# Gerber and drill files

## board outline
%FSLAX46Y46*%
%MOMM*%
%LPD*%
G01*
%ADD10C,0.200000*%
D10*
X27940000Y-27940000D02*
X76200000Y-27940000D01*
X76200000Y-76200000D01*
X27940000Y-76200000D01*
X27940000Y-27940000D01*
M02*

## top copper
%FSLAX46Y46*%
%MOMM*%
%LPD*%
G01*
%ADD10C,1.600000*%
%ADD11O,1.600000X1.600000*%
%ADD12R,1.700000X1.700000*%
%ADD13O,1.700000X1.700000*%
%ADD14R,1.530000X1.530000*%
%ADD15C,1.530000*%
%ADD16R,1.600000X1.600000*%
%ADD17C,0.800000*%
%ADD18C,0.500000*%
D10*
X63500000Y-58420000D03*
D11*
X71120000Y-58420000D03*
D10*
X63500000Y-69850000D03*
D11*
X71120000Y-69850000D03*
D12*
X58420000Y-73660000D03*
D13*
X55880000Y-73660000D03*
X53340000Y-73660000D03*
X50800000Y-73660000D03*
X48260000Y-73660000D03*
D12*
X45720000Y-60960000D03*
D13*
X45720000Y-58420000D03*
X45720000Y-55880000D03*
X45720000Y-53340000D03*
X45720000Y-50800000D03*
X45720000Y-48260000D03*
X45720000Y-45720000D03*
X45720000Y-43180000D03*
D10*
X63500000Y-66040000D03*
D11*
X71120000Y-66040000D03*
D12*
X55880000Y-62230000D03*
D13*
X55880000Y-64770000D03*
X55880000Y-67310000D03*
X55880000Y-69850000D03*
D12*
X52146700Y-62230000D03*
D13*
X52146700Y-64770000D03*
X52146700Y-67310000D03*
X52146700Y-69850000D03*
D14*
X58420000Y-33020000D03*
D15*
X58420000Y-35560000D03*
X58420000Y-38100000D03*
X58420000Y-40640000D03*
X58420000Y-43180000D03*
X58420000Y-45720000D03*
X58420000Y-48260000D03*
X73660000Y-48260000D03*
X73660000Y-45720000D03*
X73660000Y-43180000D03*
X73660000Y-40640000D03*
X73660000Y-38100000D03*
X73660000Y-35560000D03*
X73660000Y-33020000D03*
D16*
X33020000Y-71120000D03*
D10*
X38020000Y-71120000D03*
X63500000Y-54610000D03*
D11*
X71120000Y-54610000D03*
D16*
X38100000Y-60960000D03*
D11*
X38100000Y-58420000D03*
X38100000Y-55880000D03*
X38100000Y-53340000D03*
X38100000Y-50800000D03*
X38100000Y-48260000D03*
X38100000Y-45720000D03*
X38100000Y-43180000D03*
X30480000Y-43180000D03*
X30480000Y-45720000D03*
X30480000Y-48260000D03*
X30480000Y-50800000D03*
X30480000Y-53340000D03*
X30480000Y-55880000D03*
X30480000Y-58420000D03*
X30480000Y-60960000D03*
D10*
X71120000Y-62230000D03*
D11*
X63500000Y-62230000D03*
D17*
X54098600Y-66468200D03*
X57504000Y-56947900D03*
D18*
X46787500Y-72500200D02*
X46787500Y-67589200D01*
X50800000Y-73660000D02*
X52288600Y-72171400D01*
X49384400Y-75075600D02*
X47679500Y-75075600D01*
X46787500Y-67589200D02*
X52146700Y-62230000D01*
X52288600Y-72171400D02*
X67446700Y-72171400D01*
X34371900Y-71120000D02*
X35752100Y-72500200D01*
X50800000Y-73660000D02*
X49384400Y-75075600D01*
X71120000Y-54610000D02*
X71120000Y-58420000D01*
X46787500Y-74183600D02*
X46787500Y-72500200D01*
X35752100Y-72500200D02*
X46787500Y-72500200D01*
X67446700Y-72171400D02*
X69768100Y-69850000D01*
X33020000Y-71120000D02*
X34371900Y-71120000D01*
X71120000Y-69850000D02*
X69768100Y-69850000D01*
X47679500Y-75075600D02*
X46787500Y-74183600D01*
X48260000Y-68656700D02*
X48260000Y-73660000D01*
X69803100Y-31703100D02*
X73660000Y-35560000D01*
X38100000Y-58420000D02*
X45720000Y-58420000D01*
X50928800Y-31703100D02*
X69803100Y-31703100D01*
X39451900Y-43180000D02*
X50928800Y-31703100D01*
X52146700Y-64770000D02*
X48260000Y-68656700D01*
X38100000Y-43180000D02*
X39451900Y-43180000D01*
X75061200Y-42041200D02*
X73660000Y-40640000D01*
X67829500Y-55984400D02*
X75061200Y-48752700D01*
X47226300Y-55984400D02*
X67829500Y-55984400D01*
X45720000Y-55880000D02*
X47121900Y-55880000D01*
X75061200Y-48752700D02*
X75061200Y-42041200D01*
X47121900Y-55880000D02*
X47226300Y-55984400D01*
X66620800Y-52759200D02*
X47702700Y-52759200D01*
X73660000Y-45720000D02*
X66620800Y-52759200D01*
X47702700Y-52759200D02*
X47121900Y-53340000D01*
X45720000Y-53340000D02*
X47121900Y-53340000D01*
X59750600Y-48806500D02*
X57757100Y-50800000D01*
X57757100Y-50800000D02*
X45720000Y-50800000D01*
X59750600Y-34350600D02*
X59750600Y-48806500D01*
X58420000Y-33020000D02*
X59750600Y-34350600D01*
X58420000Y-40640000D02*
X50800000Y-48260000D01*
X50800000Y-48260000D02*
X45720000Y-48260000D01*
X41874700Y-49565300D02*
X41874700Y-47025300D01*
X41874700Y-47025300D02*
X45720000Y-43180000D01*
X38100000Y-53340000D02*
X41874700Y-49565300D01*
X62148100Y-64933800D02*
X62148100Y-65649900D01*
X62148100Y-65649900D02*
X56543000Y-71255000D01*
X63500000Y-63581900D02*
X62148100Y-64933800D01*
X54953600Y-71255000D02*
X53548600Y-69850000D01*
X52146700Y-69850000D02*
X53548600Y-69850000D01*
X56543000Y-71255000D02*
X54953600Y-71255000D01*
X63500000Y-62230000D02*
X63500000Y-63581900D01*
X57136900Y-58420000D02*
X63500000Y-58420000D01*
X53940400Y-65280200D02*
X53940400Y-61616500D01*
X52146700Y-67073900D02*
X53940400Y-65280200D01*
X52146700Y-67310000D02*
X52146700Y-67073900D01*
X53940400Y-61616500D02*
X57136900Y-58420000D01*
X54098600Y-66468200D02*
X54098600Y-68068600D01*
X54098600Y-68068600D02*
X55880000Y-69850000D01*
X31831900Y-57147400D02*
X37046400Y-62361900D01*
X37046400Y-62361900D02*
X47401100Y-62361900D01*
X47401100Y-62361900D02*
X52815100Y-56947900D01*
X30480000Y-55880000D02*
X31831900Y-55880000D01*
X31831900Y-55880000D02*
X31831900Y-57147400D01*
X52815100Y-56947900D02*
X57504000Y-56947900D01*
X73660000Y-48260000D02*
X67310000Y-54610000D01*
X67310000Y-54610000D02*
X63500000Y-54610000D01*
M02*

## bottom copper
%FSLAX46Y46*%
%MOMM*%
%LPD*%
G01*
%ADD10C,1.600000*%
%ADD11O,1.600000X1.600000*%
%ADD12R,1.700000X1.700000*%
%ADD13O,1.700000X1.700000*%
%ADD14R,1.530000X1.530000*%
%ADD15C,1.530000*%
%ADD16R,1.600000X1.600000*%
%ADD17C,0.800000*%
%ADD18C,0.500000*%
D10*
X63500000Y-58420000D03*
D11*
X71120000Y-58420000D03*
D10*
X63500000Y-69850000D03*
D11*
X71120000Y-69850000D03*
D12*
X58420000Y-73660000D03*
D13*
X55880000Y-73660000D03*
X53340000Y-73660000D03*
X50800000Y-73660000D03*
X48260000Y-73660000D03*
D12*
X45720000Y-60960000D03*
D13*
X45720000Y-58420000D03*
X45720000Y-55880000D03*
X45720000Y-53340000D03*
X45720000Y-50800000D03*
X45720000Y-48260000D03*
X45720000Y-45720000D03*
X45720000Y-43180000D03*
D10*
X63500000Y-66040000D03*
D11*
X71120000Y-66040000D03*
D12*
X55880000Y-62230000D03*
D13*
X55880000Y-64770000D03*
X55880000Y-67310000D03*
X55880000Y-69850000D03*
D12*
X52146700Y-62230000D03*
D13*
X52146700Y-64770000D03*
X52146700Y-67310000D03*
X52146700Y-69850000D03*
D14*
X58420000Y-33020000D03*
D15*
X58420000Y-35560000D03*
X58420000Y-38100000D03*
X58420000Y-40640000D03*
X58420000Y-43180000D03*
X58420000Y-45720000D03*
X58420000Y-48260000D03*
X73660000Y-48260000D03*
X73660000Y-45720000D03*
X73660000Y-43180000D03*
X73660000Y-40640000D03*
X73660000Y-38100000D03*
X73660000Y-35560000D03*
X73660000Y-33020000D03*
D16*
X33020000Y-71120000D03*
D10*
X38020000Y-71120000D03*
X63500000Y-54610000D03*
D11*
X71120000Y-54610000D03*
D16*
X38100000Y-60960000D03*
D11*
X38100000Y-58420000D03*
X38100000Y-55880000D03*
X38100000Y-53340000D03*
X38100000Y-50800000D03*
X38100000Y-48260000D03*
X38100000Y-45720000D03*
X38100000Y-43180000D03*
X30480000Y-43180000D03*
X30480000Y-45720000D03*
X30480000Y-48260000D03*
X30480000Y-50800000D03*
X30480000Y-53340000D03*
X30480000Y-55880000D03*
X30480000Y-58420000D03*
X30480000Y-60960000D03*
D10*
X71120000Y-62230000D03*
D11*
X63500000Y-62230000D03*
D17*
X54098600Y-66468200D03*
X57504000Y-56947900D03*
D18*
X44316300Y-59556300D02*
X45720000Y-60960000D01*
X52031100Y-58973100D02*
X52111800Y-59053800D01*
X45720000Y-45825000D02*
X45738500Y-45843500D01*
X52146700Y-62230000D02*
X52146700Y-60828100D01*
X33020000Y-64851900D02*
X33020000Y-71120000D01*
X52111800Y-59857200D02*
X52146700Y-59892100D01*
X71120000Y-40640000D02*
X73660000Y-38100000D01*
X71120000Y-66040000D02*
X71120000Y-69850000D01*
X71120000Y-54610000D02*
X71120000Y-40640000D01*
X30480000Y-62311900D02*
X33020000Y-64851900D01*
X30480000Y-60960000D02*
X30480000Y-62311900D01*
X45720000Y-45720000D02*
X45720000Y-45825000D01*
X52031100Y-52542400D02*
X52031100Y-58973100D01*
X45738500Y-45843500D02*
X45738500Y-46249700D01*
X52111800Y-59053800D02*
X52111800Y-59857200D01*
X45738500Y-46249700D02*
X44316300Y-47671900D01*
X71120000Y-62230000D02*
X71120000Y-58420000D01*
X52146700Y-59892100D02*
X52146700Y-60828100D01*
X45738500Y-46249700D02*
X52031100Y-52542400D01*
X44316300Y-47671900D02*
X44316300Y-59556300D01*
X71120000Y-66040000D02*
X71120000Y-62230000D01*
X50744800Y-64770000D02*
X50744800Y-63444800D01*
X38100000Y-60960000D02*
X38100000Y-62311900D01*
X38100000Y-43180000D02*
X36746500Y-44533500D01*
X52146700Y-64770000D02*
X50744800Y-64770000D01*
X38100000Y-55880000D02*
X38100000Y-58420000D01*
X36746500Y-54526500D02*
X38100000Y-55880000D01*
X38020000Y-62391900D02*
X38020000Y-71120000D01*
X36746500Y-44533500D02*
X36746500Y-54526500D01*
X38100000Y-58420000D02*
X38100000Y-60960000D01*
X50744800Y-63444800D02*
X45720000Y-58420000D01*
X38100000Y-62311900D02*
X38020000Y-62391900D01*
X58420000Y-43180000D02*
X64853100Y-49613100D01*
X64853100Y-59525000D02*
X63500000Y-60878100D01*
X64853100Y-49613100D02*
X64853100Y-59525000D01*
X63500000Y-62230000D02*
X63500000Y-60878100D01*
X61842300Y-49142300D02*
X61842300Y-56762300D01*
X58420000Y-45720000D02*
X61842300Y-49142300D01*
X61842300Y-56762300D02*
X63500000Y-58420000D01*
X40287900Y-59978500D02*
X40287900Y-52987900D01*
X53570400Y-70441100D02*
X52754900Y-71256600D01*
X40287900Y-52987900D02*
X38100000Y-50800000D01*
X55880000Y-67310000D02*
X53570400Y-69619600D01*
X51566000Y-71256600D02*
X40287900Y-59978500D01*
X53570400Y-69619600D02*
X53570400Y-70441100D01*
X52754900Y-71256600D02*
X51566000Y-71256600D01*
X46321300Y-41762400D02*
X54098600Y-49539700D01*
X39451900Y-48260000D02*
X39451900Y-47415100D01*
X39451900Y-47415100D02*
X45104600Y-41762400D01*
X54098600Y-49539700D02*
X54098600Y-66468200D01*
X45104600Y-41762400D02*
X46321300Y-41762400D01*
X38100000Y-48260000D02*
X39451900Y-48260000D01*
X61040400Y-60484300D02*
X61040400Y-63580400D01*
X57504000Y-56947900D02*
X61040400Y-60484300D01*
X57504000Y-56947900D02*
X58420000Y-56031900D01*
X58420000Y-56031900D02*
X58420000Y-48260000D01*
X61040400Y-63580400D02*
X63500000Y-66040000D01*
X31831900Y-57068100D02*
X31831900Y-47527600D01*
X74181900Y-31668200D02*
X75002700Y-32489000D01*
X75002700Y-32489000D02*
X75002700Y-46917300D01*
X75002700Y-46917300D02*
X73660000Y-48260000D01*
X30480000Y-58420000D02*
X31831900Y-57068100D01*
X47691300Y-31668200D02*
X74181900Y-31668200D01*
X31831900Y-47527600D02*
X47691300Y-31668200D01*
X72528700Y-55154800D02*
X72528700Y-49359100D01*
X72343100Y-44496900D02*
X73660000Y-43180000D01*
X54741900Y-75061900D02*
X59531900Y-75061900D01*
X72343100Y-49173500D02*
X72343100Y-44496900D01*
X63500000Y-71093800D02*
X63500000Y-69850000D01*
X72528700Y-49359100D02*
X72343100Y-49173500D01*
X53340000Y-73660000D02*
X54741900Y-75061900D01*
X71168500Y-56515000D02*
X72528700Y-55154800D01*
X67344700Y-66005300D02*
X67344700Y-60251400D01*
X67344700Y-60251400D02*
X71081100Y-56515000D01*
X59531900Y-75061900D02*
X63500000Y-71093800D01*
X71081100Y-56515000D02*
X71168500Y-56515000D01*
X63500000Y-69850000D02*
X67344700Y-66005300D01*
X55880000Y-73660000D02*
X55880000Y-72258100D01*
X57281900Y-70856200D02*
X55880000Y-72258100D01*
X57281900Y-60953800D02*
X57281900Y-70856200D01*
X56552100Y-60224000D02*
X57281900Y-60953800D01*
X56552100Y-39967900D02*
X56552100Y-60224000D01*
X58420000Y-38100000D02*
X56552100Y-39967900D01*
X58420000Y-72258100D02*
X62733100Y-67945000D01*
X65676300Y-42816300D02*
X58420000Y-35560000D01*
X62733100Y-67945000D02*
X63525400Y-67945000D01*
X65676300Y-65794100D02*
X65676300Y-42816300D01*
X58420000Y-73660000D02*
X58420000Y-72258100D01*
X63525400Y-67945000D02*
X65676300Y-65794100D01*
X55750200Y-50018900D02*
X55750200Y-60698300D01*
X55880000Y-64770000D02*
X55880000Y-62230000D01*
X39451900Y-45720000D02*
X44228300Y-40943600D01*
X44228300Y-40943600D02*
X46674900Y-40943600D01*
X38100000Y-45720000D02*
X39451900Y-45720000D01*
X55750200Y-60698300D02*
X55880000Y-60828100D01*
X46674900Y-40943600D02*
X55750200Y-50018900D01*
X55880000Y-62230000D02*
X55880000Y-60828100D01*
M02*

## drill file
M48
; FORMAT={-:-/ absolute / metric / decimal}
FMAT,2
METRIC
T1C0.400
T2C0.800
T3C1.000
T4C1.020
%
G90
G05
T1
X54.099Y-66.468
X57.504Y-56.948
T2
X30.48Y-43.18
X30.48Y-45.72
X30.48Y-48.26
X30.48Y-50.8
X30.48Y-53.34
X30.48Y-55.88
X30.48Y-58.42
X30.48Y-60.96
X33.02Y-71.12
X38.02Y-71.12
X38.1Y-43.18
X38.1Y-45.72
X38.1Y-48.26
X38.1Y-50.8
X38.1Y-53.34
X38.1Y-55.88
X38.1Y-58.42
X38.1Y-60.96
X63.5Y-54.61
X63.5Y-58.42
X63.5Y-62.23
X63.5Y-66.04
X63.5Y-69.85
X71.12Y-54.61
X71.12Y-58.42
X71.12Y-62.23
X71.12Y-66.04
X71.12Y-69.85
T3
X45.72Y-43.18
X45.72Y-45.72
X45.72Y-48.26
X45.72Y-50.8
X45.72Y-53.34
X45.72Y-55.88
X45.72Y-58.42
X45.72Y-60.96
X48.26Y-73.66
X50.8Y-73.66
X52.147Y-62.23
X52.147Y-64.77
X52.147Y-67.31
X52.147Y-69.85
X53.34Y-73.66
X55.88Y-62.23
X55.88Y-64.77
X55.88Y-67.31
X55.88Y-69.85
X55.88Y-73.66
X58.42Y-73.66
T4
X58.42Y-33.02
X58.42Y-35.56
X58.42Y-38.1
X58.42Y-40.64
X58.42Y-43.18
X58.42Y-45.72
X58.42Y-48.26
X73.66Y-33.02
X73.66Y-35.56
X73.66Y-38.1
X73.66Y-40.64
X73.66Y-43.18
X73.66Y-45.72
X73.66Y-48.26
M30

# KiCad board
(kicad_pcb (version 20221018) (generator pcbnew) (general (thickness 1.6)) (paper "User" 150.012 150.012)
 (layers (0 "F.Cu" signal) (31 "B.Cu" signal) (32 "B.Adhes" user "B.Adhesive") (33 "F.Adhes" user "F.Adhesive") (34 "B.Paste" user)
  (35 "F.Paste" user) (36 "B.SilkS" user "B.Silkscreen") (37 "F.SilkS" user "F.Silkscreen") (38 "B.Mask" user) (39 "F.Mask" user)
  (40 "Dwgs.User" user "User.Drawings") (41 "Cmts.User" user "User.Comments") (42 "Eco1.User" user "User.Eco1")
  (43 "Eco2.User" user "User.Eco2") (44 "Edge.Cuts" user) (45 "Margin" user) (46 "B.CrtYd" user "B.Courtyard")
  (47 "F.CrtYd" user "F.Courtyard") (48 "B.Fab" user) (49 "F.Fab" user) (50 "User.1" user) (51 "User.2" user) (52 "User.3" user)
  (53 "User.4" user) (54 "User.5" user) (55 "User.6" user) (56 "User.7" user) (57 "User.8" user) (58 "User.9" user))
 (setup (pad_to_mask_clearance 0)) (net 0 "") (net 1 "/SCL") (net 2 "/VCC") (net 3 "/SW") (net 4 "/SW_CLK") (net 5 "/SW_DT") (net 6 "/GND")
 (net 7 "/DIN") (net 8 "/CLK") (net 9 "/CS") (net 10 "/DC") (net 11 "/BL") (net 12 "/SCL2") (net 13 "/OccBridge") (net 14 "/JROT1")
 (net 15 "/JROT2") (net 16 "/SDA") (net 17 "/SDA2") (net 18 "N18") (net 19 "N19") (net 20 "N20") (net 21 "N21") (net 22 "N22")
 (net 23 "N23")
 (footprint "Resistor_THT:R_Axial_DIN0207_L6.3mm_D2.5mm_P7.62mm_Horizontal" (layer "F.Cu") (at 63.5 58.42)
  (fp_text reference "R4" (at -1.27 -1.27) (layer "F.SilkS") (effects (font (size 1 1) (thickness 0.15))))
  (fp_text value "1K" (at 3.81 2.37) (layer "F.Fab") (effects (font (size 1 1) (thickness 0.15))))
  (pad "1" thru_hole circle (at 0 0) (size 1.6 1.6) (drill 0.8) (layers "*.Cu" "*.Mask") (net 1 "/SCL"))
  (pad "2" thru_hole oval (at 7.62 0) (size 1.6 1.6) (drill 0.8) (layers "*.Cu" "*.Mask") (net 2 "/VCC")))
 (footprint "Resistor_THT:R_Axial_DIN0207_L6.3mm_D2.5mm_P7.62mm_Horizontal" (layer "F.Cu") (at 63.5 69.85)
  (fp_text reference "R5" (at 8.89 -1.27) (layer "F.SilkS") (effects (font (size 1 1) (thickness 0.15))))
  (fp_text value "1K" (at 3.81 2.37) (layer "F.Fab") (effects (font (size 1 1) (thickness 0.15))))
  (pad "1" thru_hole circle (at 0 0) (size 1.6 1.6) (drill 0.8) (layers "*.Cu" "*.Mask") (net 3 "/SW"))
  (pad "2" thru_hole oval (at 7.62 0) (size 1.6 1.6) (drill 0.8) (layers "*.Cu" "*.Mask") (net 2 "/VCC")))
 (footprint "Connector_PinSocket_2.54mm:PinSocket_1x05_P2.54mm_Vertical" (layer "F.Cu") (at 58.42 73.66 -90)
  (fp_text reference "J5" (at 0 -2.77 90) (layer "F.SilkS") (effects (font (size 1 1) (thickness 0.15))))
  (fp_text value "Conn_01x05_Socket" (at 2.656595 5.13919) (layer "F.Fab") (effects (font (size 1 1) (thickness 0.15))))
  (pad "1" thru_hole rect (at 0 0 270) (size 1.7 1.7) (drill 1) (layers "*.Cu" "*.Mask") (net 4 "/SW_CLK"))
  (pad "2" thru_hole oval (at 0 2.54 270) (size 1.7 1.7) (drill 1) (layers "*.Cu" "*.Mask") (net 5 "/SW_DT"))
  (pad "3" thru_hole oval (at 0 5.08 270) (size 1.7 1.7) (drill 1) (layers "*.Cu" "*.Mask") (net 3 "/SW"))
  (pad "4" thru_hole oval (at 0 7.62 270) (size 1.7 1.7) (drill 1) (layers "*.Cu" "*.Mask") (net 2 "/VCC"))
  (pad "5" thru_hole oval (at 0 10.16 270) (size 1.7 1.7) (drill 1) (layers "*.Cu" "*.Mask") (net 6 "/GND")))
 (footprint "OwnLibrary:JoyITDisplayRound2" (layer "F.Cu") (at 52.13 52.07 90)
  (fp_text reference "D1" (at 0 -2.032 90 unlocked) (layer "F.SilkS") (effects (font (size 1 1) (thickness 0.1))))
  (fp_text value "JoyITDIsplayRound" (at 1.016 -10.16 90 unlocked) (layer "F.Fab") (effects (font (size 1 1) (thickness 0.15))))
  (pad "1" thru_hole rect (at -8.89 -6.41 180) (size 1.7 1.7) (drill 1) (layers "*.Cu" "*.Mask") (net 2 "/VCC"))
  (pad "2" thru_hole oval (at -6.35 -6.41 180) (size 1.7 1.7) (drill 1) (layers "*.Cu" "*.Mask") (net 6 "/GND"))
  (pad "3" thru_hole oval (at -3.81 -6.41 180) (size 1.7 1.7) (drill 1) (layers "*.Cu" "*.Mask") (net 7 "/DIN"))
  (pad "4" thru_hole oval (at -1.27 -6.41 180) (size 1.7 1.7) (drill 1) (layers "*.Cu" "*.Mask") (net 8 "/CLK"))
  (pad "5" thru_hole oval (at 1.27 -6.41 180) (size 1.7 1.7) (drill 1) (layers "*.Cu" "*.Mask") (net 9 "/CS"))
  (pad "6" thru_hole oval (at 3.81 -6.41 180) (size 1.7 1.7) (drill 1) (layers "*.Cu" "*.Mask") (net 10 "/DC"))
  (pad "7" thru_hole oval (at 6.35 -6.41 180) (size 1.7 1.7) (drill 1) (layers "*.Cu" "*.Mask") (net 2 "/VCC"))
  (pad "8" thru_hole oval (at 8.89 -6.41 180) (size 1.7 1.7) (drill 1) (layers "*.Cu" "*.Mask") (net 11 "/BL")))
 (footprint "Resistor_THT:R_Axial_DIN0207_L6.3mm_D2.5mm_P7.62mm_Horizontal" (layer "F.Cu") (at 63.5 66.04)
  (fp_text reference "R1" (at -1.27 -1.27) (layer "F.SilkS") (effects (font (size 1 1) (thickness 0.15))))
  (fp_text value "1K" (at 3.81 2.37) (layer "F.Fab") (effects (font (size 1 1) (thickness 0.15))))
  (pad "1" thru_hole circle (at 0 0) (size 1.6 1.6) (drill 0.8) (layers "*.Cu" "*.Mask") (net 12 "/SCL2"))
  (pad "2" thru_hole oval (at 7.62 0) (size 1.6 1.6) (drill 0.8) (layers "*.Cu" "*.Mask") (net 2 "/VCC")))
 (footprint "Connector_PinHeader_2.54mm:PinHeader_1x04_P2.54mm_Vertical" (layer "F.Cu") (at 55.88 62.23)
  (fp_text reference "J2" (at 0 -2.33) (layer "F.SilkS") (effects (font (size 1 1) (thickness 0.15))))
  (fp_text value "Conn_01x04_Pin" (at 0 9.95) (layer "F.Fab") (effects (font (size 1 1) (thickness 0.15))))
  (pad "1" thru_hole rect (at 0 0) (size 1.7 1.7) (drill 1) (layers "*.Cu" "*.Mask") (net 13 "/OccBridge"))
  (pad "2" thru_hole oval (at 0 2.54) (size 1.7 1.7) (drill 1) (layers "*.Cu" "*.Mask") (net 13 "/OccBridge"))
  (pad "3" thru_hole oval (at 0 5.08) (size 1.7 1.7) (drill 1) (layers "*.Cu" "*.Mask") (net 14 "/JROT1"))
  (pad "4" thru_hole oval (at 0 7.62) (size 1.7 1.7) (drill 1) (layers "*.Cu" "*.Mask") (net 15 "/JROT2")))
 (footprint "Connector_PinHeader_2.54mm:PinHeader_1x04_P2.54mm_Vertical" (layer "F.Cu") (at 52.1467 62.23)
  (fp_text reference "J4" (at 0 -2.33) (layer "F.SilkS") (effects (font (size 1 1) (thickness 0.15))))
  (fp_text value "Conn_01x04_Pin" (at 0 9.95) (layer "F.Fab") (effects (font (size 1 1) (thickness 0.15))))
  (pad "1" thru_hole rect (at 0 0) (size 1.7 1.7) (drill 1) (layers "*.Cu" "*.Mask") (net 2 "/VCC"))
  (pad "2" thru_hole oval (at 0 2.54) (size 1.7 1.7) (drill 1) (layers "*.Cu" "*.Mask") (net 6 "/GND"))
  (pad "3" thru_hole oval (at 0 5.08) (size 1.7 1.7) (drill 1) (layers "*.Cu" "*.Mask") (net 1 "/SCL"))
  (pad "4" thru_hole oval (at 0 7.62) (size 1.7 1.7) (drill 1) (layers "*.Cu" "*.Mask") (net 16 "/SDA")))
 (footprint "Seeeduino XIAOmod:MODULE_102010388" (layer "F.Cu") (at 66.04 40.64)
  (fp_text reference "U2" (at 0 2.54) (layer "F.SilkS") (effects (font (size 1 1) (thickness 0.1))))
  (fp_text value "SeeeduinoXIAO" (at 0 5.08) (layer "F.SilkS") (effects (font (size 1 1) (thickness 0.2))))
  (pad "1" thru_hole rect (at -7.62 -7.62) (size 1.53 1.53) (drill 1.02) (layers "*.Cu" "*.Mask") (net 9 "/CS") (thermal_bridge_angle 45))
  (pad "2" thru_hole circle (at -7.62 -5.08) (size 1.53 1.53) (drill 1.02) (layers "*.Cu" "*.Mask") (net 4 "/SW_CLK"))
  (pad "3" thru_hole circle (at -7.62 -2.54) (size 1.53 1.53) (drill 1.02) (layers "*.Cu" "*.Mask") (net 5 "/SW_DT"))
  (pad "4" thru_hole circle (at -7.62 0) (size 1.53 1.53) (drill 1.02) (layers "*.Cu" "*.Mask") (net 10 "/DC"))
  (pad "5" thru_hole circle (at -7.62 2.54) (size 1.53 1.53) (drill 1.02) (layers "*.Cu" "*.Mask") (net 16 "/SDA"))
  (pad "6" thru_hole circle (at -7.62 5.08) (size 1.53 1.53) (drill 1.02) (layers "*.Cu" "*.Mask") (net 1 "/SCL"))
  (pad "7" thru_hole circle (at -7.62 7.62) (size 1.53 1.53) (drill 1.02) (layers "*.Cu" "*.Mask") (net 12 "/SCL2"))
  (pad "8" thru_hole circle (at 7.62 7.62) (size 1.53 1.53) (drill 1.02) (layers "*.Cu" "*.Mask") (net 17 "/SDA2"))
  (pad "9" thru_hole circle (at 7.62 5.08) (size 1.53 1.53) (drill 1.02) (layers "*.Cu" "*.Mask") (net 8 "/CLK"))
  (pad "10" thru_hole circle (at 7.62 2.54) (size 1.53 1.53) (drill 1.02) (layers "*.Cu" "*.Mask") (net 3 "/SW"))
  (pad "11" thru_hole circle (at 7.62 0) (size 1.53 1.53) (drill 1.02) (layers "*.Cu" "*.Mask") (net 7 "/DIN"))
  (pad "12" thru_hole circle (at 7.62 -2.54) (size 1.53 1.53) (drill 1.02) (layers "*.Cu" "*.Mask") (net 2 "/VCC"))
  (pad "13" thru_hole circle (at 7.62 -5.08) (size 1.53 1.53) (drill 1.02) (layers "*.Cu" "*.Mask") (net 6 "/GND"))
  (pad "14" thru_hole circle (at 7.62 -7.62) (size 1.53 1.53) (drill 1.02) (layers "*.Cu" "*.Mask") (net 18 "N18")))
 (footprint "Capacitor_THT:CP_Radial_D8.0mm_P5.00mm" (layer "F.Cu") (at 33.02 71.12)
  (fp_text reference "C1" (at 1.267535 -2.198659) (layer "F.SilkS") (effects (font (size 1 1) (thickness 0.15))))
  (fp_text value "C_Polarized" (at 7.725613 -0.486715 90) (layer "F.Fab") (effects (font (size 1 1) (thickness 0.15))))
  (pad "1" thru_hole rect (at 0 0) (size 1.6 1.6) (drill 0.8) (layers "*.Cu" "*.Mask") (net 2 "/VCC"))
  (pad "2" thru_hole circle (at 5 0) (size 1.6 1.6) (drill 0.8) (layers "*.Cu" "*.Mask") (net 6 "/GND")))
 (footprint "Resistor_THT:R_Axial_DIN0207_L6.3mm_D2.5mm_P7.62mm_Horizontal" (layer "F.Cu") (at 63.5 54.61)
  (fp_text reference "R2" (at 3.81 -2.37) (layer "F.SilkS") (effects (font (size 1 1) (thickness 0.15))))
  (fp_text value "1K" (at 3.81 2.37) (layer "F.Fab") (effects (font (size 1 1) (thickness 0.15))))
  (pad "1" thru_hole circle (at 0 0) (size 1.6 1.6) (drill 0.8) (layers "*.Cu" "*.Mask") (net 17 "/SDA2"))
  (pad "2" thru_hole oval (at 7.62 0) (size 1.6 1.6) (drill 0.8) (layers "*.Cu" "*.Mask") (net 2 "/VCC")))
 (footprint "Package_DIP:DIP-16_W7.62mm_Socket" (layer "F.Cu") (at 38.1 60.96 180)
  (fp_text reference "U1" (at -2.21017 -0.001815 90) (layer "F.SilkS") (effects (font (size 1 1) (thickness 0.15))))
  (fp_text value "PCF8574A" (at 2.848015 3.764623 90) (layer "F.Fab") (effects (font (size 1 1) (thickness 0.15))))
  (pad "1" thru_hole rect (at 0 0 180) (size 1.6 1.6) (drill 0.8) (layers "*.Cu" "*.Mask") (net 6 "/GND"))
  (pad "2" thru_hole oval (at 0 2.54 180) (size 1.6 1.6) (drill 0.8) (layers "*.Cu" "*.Mask") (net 6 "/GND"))
  (pad "3" thru_hole oval (at 0 5.08 180) (size 1.6 1.6) (drill 0.8) (layers "*.Cu" "*.Mask") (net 6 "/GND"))
  (pad "4" thru_hole oval (at 0 7.62 180) (size 1.6 1.6) (drill 0.8) (layers "*.Cu" "*.Mask") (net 11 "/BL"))
  (pad "5" thru_hole oval (at 0 10.16 180) (size 1.6 1.6) (drill 0.8) (layers "*.Cu" "*.Mask") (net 14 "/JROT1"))
  (pad "6" thru_hole oval (at 0 12.7 180) (size 1.6 1.6) (drill 0.8) (layers "*.Cu" "*.Mask") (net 15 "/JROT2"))
  (pad "7" thru_hole oval (at 0 15.24 180) (size 1.6 1.6) (drill 0.8) (layers "*.Cu" "*.Mask") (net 13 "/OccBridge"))
  (pad "8" thru_hole oval (at 0 17.78 180) (size 1.6 1.6) (drill 0.8) (layers "*.Cu" "*.Mask") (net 6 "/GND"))
  (pad "9" thru_hole oval (at 7.62 17.78 180) (size 1.6 1.6) (drill 0.8) (layers "*.Cu" "*.Mask") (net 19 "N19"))
  (pad "10" thru_hole oval (at 7.62 15.24 180) (size 1.6 1.6) (drill 0.8) (layers "*.Cu" "*.Mask") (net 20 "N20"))
  (pad "11" thru_hole oval (at 7.62 12.7 180) (size 1.6 1.6) (drill 0.8) (layers "*.Cu" "*.Mask") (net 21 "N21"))
  (pad "12" thru_hole oval (at 7.62 10.16 180) (size 1.6 1.6) (drill 0.8) (layers "*.Cu" "*.Mask") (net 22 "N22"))
  (pad "13" thru_hole oval (at 7.62 7.62 180) (size 1.6 1.6) (drill 0.8) (layers "*.Cu" "*.Mask") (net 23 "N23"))
  (pad "14" thru_hole oval (at 7.62 5.08 180) (size 1.6 1.6) (drill 0.8) (layers "*.Cu" "*.Mask") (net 12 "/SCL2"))
  (pad "15" thru_hole oval (at 7.62 2.54 180) (size 1.6 1.6) (drill 0.8) (layers "*.Cu" "*.Mask") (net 17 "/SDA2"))
  (pad "16" thru_hole oval (at 7.62 0 180) (size 1.6 1.6) (drill 0.8) (layers "*.Cu" "*.Mask") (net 2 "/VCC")))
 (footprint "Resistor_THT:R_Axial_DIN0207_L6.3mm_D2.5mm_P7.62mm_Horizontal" (layer "F.Cu") (at 71.12 62.23 180)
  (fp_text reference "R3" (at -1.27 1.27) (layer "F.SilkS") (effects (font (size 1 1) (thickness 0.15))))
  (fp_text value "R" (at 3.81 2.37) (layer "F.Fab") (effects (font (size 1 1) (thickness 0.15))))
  (pad "1" thru_hole circle (at 0 0 180) (size 1.6 1.6) (drill 0.8) (layers "*.Cu" "*.Mask") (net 2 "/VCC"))
  (pad "2" thru_hole oval (at 7.62 0 180) (size 1.6 1.6) (drill 0.8) (layers "*.Cu" "*.Mask") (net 16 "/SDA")))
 (gr_rect locked (start 27.94 27.94) (end 76.2 76.2) (stroke (width 0.2) (type default)) (fill none) (layer "Edge.Cuts"))
 (segment (start 46.7875 72.5002) (end 46.7875 67.5892) (width 0.5) (layer "F.Cu") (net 2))
 (segment (start 50.8 73.66) (end 52.2886 72.1714) (width 0.5) (layer "F.Cu") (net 2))
 (segment (start 49.3844 75.0756) (end 47.6795 75.0756) (width 0.5) (layer "F.Cu") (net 2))
 (segment (start 46.7875 67.5892) (end 52.1467 62.23) (width 0.5) (layer "F.Cu") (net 2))
 (segment (start 52.2886 72.1714) (end 67.4467 72.1714) (width 0.5) (layer "F.Cu") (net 2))
 (segment (start 34.3719 71.12) (end 35.7521 72.5002) (width 0.5) (layer "F.Cu") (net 2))
 (segment (start 50.8 73.66) (end 49.3844 75.0756) (width 0.5) (layer "F.Cu") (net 2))
 (segment (start 71.12 54.61) (end 71.12 58.42) (width 0.5) (layer "F.Cu") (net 2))
 (segment (start 46.7875 74.1836) (end 46.7875 72.5002) (width 0.5) (layer "F.Cu") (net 2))
 (segment (start 35.7521 72.5002) (end 46.7875 72.5002) (width 0.5) (layer "F.Cu") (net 2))
 (segment (start 67.4467 72.1714) (end 69.7681 69.85) (width 0.5) (layer "F.Cu") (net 2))
 (segment (start 33.02 71.12) (end 34.3719 71.12) (width 0.5) (layer "F.Cu") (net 2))
 (segment (start 71.12 69.85) (end 69.7681 69.85) (width 0.5) (layer "F.Cu") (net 2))
 (segment (start 47.6795 75.0756) (end 46.7875 74.1836) (width 0.5) (layer "F.Cu") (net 2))
 (segment (start 44.3163 59.5563) (end 45.72 60.96) (width 0.5) (layer "B.Cu") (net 2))
 (segment (start 52.0311 58.9731) (end 52.1118 59.0538) (width 0.5) (layer "B.Cu") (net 2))
 (segment (start 45.72 45.825) (end 45.7385 45.8435) (width 0.5) (layer "B.Cu") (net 2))
 (segment (start 52.1467 62.23) (end 52.1467 60.8281) (width 0.5) (layer "B.Cu") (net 2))
 (segment (start 33.02 64.8519) (end 33.02 71.12) (width 0.5) (layer "B.Cu") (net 2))
 (segment (start 52.1118 59.8572) (end 52.1467 59.8921) (width 0.5) (layer "B.Cu") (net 2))
 (segment (start 71.12 40.64) (end 73.66 38.1) (width 0.5) (layer "B.Cu") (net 2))
 (segment (start 71.12 66.04) (end 71.12 69.85) (width 0.5) (layer "B.Cu") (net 2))
 (segment (start 71.12 54.61) (end 71.12 40.64) (width 0.5) (layer "B.Cu") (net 2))
 (segment (start 30.48 62.3119) (end 33.02 64.8519) (width 0.5) (layer "B.Cu") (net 2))
 (segment (start 30.48 60.96) (end 30.48 62.3119) (width 0.5) (layer "B.Cu") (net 2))
 (segment (start 45.72 45.72) (end 45.72 45.825) (width 0.5) (layer "B.Cu") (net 2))
 (segment (start 52.0311 52.5424) (end 52.0311 58.9731) (width 0.5) (layer "B.Cu") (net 2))
 (segment (start 45.7385 45.8435) (end 45.7385 46.2497) (width 0.5) (layer "B.Cu") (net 2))
 (segment (start 52.1118 59.0538) (end 52.1118 59.8572) (width 0.5) (layer "B.Cu") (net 2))
 (segment (start 45.7385 46.2497) (end 44.3163 47.6719) (width 0.5) (layer "B.Cu") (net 2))
 (segment (start 71.12 62.23) (end 71.12 58.42) (width 0.5) (layer "B.Cu") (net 2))
 (segment (start 52.1467 59.8921) (end 52.1467 60.8281) (width 0.5) (layer "B.Cu") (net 2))
 (segment (start 45.7385 46.2497) (end 52.0311 52.5424) (width 0.5) (layer "B.Cu") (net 2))
 (segment (start 44.3163 47.6719) (end 44.3163 59.5563) (width 0.5) (layer "B.Cu") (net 2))
 (segment (start 71.12 66.04) (end 71.12 62.23) (width 0.5) (layer "B.Cu") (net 2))
 (segment (start 48.26 68.6567) (end 48.26 73.66) (width 0.5) (layer "F.Cu") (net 6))
 (segment (start 69.8031 31.7031) (end 73.66 35.56) (width 0.5) (layer "F.Cu") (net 6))
 (segment (start 38.1 58.42) (end 45.72 58.42) (width 0.5) (layer "F.Cu") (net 6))
 (segment (start 50.9288 31.7031) (end 69.8031 31.7031) (width 0.5) (layer "F.Cu") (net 6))
 (segment (start 39.4519 43.18) (end 50.9288 31.7031) (width 0.5) (layer "F.Cu") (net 6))
 (segment (start 52.1467 64.77) (end 48.26 68.6567) (width 0.5) (layer "F.Cu") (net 6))
 (segment (start 38.1 43.18) (end 39.4519 43.18) (width 0.5) (layer "F.Cu") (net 6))
 (segment (start 50.7448 64.77) (end 50.7448 63.4448) (width 0.5) (layer "B.Cu") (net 6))
 (segment (start 38.1 60.96) (end 38.1 62.3119) (width 0.5) (layer "B.Cu") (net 6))
 (segment (start 38.1 43.18) (end 36.7465 44.5335) (width 0.5) (layer "B.Cu") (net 6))
 (segment (start 52.1467 64.77) (end 50.7448 64.77) (width 0.5) (layer "B.Cu") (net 6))
 (segment (start 38.1 55.88) (end 38.1 58.42) (width 0.5) (layer "B.Cu") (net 6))
 (segment (start 36.7465 54.5265) (end 38.1 55.88) (width 0.5) (layer "B.Cu") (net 6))
 (segment (start 38.02 62.3919) (end 38.02 71.12) (width 0.5) (layer "B.Cu") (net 6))
 (segment (start 36.7465 44.5335) (end 36.7465 54.5265) (width 0.5) (layer "B.Cu") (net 6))
 (segment (start 38.1 58.42) (end 38.1 60.96) (width 0.5) (layer "B.Cu") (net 6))
 (segment (start 50.7448 63.4448) (end 45.72 58.42) (width 0.5) (layer "B.Cu") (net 6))
 (segment (start 38.1 62.3119) (end 38.02 62.3919) (width 0.5) (layer "B.Cu") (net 6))
 (segment (start 75.0612 42.0412) (end 73.66 40.64) (width 0.5) (layer "F.Cu") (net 7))
 (segment (start 67.8295 55.9844) (end 75.0612 48.7527) (width 0.5) (layer "F.Cu") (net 7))
 (segment (start 47.2263 55.9844) (end 67.8295 55.9844) (width 0.5) (layer "F.Cu") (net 7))
 (segment (start 45.72 55.88) (end 47.1219 55.88) (width 0.5) (layer "F.Cu") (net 7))
 (segment (start 75.0612 48.7527) (end 75.0612 42.0412) (width 0.5) (layer "F.Cu") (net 7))
 (segment (start 47.1219 55.88) (end 47.2263 55.9844) (width 0.5) (layer "F.Cu") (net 7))
 (segment (start 66.6208 52.7592) (end 47.7027 52.7592) (width 0.5) (layer "F.Cu") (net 8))
 (segment (start 73.66 45.72) (end 66.6208 52.7592) (width 0.5) (layer "F.Cu") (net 8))
 (segment (start 47.7027 52.7592) (end 47.1219 53.34) (width 0.5) (layer "F.Cu") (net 8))
 (segment (start 45.72 53.34) (end 47.1219 53.34) (width 0.5) (layer "F.Cu") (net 8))
 (segment (start 59.7506 48.8065) (end 57.7571 50.8) (width 0.5) (layer "F.Cu") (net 9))
 (segment (start 57.7571 50.8) (end 45.72 50.8) (width 0.5) (layer "F.Cu") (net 9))
 (segment (start 59.7506 34.3506) (end 59.7506 48.8065) (width 0.5) (layer "F.Cu") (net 9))
 (segment (start 58.42 33.02) (end 59.7506 34.3506) (width 0.5) (layer "F.Cu") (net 9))
 (segment (start 58.42 40.64) (end 50.8 48.26) (width 0.5) (layer "F.Cu") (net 10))
 (segment (start 50.8 48.26) (end 45.72 48.26) (width 0.5) (layer "F.Cu") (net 10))
 (segment (start 41.8747 49.5653) (end 41.8747 47.0253) (width 0.5) (layer "F.Cu") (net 11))
 (segment (start 41.8747 47.0253) (end 45.72 43.18) (width 0.5) (layer "F.Cu") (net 11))
 (segment (start 38.1 53.34) (end 41.8747 49.5653) (width 0.5) (layer "F.Cu") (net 11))
 (segment (start 62.1481 64.9338) (end 62.1481 65.6499) (width 0.5) (layer "F.Cu") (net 16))
 (segment (start 62.1481 65.6499) (end 56.543 71.255) (width 0.5) (layer "F.Cu") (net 16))
 (segment (start 63.5 63.5819) (end 62.1481 64.9338) (width 0.5) (layer "F.Cu") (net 16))
 (segment (start 54.9536 71.255) (end 53.5486 69.85) (width 0.5) (layer "F.Cu") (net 16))
 (segment (start 52.1467 69.85) (end 53.5486 69.85) (width 0.5) (layer "F.Cu") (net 16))
 (segment (start 56.543 71.255) (end 54.9536 71.255) (width 0.5) (layer "F.Cu") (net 16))
 (segment (start 63.5 62.23) (end 63.5 63.5819) (width 0.5) (layer "F.Cu") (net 16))
 (segment (start 58.42 43.18) (end 64.8531 49.6131) (width 0.5) (layer "B.Cu") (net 16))
 (segment (start 64.8531 59.525) (end 63.5 60.8781) (width 0.5) (layer "B.Cu") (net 16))
 (segment (start 64.8531 49.6131) (end 64.8531 59.525) (width 0.5) (layer "B.Cu") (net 16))
 (segment (start 63.5 62.23) (end 63.5 60.8781) (width 0.5) (layer "B.Cu") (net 16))
 (segment (start 57.1369 58.42) (end 63.5 58.42) (width 0.5) (layer "F.Cu") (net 1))
 (segment (start 53.9404 65.2802) (end 53.9404 61.6165) (width 0.5) (layer "F.Cu") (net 1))
 (segment (start 52.1467 67.0739) (end 53.9404 65.2802) (width 0.5) (layer "F.Cu") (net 1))
 (segment (start 52.1467 67.31) (end 52.1467 67.0739) (width 0.5) (layer "F.Cu") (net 1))
 (segment (start 53.9404 61.6165) (end 57.1369 58.42) (width 0.5) (layer "F.Cu") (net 1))
 (segment (start 61.8423 49.1423) (end 61.8423 56.7623) (width 0.5) (layer "B.Cu") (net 1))
 (segment (start 58.42 45.72) (end 61.8423 49.1423) (width 0.5) (layer "B.Cu") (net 1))
 (segment (start 61.8423 56.7623) (end 63.5 58.42) (width 0.5) (layer "B.Cu") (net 1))
 (segment (start 40.2879 59.9785) (end 40.2879 52.9879) (width 0.5) (layer "B.Cu") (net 14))
 (segment (start 53.5704 70.4411) (end 52.7549 71.2566) (width 0.5) (layer "B.Cu") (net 14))
 (segment (start 40.2879 52.9879) (end 38.1 50.8) (width 0.5) (layer "B.Cu") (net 14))
 (segment (start 55.88 67.31) (end 53.5704 69.6196) (width 0.5) (layer "B.Cu") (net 14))
 (segment (start 51.566 71.2566) (end 40.2879 59.9785) (width 0.5) (layer "B.Cu") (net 14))
 (segment (start 53.5704 69.6196) (end 53.5704 70.4411) (width 0.5) (layer "B.Cu") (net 14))
 (segment (start 52.7549 71.2566) (end 51.566 71.2566) (width 0.5) (layer "B.Cu") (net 14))
 (segment (start 54.0986 66.4682) (end 54.0986 68.0686) (width 0.5) (layer "F.Cu") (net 15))
 (segment (start 54.0986 68.0686) (end 55.88 69.85) (width 0.5) (layer "F.Cu") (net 15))
 (via (at 54.0986 66.4682) (size 0.8) (drill 0.4) (layers "F.Cu" "B.Cu") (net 15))
 (segment (start 46.3213 41.7624) (end 54.0986 49.5397) (width 0.5) (layer "B.Cu") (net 15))
 (segment (start 39.4519 48.26) (end 39.4519 47.4151) (width 0.5) (layer "B.Cu") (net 15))
 (segment (start 39.4519 47.4151) (end 45.1046 41.7624) (width 0.5) (layer "B.Cu") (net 15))
 (segment (start 54.0986 49.5397) (end 54.0986 66.4682) (width 0.5) (layer "B.Cu") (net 15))
 (segment (start 45.1046 41.7624) (end 46.3213 41.7624) (width 0.5) (layer "B.Cu") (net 15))
 (segment (start 38.1 48.26) (end 39.4519 48.26) (width 0.5) (layer "B.Cu") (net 15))
 (segment (start 31.8319 57.1474) (end 37.0464 62.3619) (width 0.5) (layer "F.Cu") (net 12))
 (segment (start 37.0464 62.3619) (end 47.4011 62.3619) (width 0.5) (layer "F.Cu") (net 12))
 (segment (start 47.4011 62.3619) (end 52.8151 56.9479) (width 0.5) (layer "F.Cu") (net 12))
 (segment (start 30.48 55.88) (end 31.8319 55.88) (width 0.5) (layer "F.Cu") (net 12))
 (segment (start 31.8319 55.88) (end 31.8319 57.1474) (width 0.5) (layer "F.Cu") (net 12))
 (segment (start 52.8151 56.9479) (end 57.504 56.9479) (width 0.5) (layer "F.Cu") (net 12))
 (via (at 57.504 56.9479) (size 0.8) (drill 0.4) (layers "F.Cu" "B.Cu") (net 12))
 (segment (start 61.0404 60.4843) (end 61.0404 63.5804) (width 0.5) (layer "B.Cu") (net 12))
 (segment (start 57.504 56.9479) (end 61.0404 60.4843) (width 0.5) (layer "B.Cu") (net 12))
 (segment (start 57.504 56.9479) (end 58.42 56.0319) (width 0.5) (layer "B.Cu") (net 12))
 (segment (start 58.42 56.0319) (end 58.42 48.26) (width 0.5) (layer "B.Cu") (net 12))
 (segment (start 61.0404 63.5804) (end 63.5 66.04) (width 0.5) (layer "B.Cu") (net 12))
 (segment (start 73.66 48.26) (end 67.31 54.61) (width 0.5) (layer "F.Cu") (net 17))
 (segment (start 67.31 54.61) (end 63.5 54.61) (width 0.5) (layer "F.Cu") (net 17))
 (segment (start 31.8319 57.0681) (end 31.8319 47.5276) (width 0.5) (layer "B.Cu") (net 17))
 (segment (start 74.1819 31.6682) (end 75.0027 32.489) (width 0.5) (layer "B.Cu") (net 17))
 (segment (start 75.0027 32.489) (end 75.0027 46.9173) (width 0.5) (layer "B.Cu") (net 17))
 (segment (start 75.0027 46.9173) (end 73.66 48.26) (width 0.5) (layer "B.Cu") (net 17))
 (segment (start 30.48 58.42) (end 31.8319 57.0681) (width 0.5) (layer "B.Cu") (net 17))
 (segment (start 47.6913 31.6682) (end 74.1819 31.6682) (width 0.5) (layer "B.Cu") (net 17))
 (segment (start 31.8319 47.5276) (end 47.6913 31.6682) (width 0.5) (layer "B.Cu") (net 17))
 (segment (start 72.5287 55.1548) (end 72.5287 49.3591) (width 0.5) (layer "B.Cu") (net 3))
 (segment (start 72.3431 44.4969) (end 73.66 43.18) (width 0.5) (layer "B.Cu") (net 3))
 (segment (start 54.7419 75.0619) (end 59.5319 75.0619) (width 0.5) (layer "B.Cu") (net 3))
 (segment (start 72.3431 49.1735) (end 72.3431 44.4969) (width 0.5) (layer "B.Cu") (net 3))
 (segment (start 63.5 71.0938) (end 63.5 69.85) (width 0.5) (layer "B.Cu") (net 3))
 (segment (start 72.5287 49.3591) (end 72.3431 49.1735) (width 0.5) (layer "B.Cu") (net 3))
 (segment (start 53.34 73.66) (end 54.7419 75.0619) (width 0.5) (layer "B.Cu") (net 3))
 (segment (start 71.1685 56.515) (end 72.5287 55.1548) (width 0.5) (layer "B.Cu") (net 3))
 (segment (start 67.3447 66.0053) (end 67.3447 60.2514) (width 0.5) (layer "B.Cu") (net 3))
 (segment (start 67.3447 60.2514) (end 71.0811 56.515) (width 0.5) (layer "B.Cu") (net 3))
 (segment (start 59.5319 75.0619) (end 63.5 71.0938) (width 0.5) (layer "B.Cu") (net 3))
 (segment (start 71.0811 56.515) (end 71.1685 56.515) (width 0.5) (layer "B.Cu") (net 3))
 (segment (start 63.5 69.85) (end 67.3447 66.0053) (width 0.5) (layer "B.Cu") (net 3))
 (segment (start 55.88 73.66) (end 55.88 72.2581) (width 0.5) (layer "B.Cu") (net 5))
 (segment (start 57.2819 70.8562) (end 55.88 72.2581) (width 0.5) (layer "B.Cu") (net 5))
 (segment (start 57.2819 60.9538) (end 57.2819 70.8562) (width 0.5) (layer "B.Cu") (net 5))
 (segment (start 56.5521 60.224) (end 57.2819 60.9538) (width 0.5) (layer "B.Cu") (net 5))
 (segment (start 56.5521 39.9679) (end 56.5521 60.224) (width 0.5) (layer "B.Cu") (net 5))
 (segment (start 58.42 38.1) (end 56.5521 39.9679) (width 0.5) (layer "B.Cu") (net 5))
 (segment (start 58.42 72.2581) (end 62.7331 67.945) (width 0.5) (layer "B.Cu") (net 4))
 (segment (start 65.6763 42.8163) (end 58.42 35.56) (width 0.5) (layer "B.Cu") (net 4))
 (segment (start 62.7331 67.945) (end 63.5254 67.945) (width 0.5) (layer "B.Cu") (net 4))
 (segment (start 65.6763 65.7941) (end 65.6763 42.8163) (width 0.5) (layer "B.Cu") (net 4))
 (segment (start 58.42 73.66) (end 58.42 72.2581) (width 0.5) (layer "B.Cu") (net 4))
 (segment (start 63.5254 67.945) (end 65.6763 65.7941) (width 0.5) (layer "B.Cu") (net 4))
 (segment (start 55.7502 50.0189) (end 55.7502 60.6983) (width 0.5) (layer "B.Cu") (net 13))
 (segment (start 55.88 64.77) (end 55.88 62.23) (width 0.5) (layer "B.Cu") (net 13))
 (segment (start 39.4519 45.72) (end 44.2283 40.9436) (width 0.5) (layer "B.Cu") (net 13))
 (segment (start 44.2283 40.9436) (end 46.6749 40.9436) (width 0.5) (layer "B.Cu") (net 13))
 (segment (start 38.1 45.72) (end 39.4519 45.72) (width 0.5) (layer "B.Cu") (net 13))
 (segment (start 55.7502 60.6983) (end 55.88 60.8281) (width 0.5) (layer "B.Cu") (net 13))
 (segment (start 46.6749 40.9436) (end 55.7502 50.0189) (width 0.5) (layer "B.Cu") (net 13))
 (segment (start 55.88 62.23) (end 55.88 60.8281) (width 0.5) (layer "B.Cu") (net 13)))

